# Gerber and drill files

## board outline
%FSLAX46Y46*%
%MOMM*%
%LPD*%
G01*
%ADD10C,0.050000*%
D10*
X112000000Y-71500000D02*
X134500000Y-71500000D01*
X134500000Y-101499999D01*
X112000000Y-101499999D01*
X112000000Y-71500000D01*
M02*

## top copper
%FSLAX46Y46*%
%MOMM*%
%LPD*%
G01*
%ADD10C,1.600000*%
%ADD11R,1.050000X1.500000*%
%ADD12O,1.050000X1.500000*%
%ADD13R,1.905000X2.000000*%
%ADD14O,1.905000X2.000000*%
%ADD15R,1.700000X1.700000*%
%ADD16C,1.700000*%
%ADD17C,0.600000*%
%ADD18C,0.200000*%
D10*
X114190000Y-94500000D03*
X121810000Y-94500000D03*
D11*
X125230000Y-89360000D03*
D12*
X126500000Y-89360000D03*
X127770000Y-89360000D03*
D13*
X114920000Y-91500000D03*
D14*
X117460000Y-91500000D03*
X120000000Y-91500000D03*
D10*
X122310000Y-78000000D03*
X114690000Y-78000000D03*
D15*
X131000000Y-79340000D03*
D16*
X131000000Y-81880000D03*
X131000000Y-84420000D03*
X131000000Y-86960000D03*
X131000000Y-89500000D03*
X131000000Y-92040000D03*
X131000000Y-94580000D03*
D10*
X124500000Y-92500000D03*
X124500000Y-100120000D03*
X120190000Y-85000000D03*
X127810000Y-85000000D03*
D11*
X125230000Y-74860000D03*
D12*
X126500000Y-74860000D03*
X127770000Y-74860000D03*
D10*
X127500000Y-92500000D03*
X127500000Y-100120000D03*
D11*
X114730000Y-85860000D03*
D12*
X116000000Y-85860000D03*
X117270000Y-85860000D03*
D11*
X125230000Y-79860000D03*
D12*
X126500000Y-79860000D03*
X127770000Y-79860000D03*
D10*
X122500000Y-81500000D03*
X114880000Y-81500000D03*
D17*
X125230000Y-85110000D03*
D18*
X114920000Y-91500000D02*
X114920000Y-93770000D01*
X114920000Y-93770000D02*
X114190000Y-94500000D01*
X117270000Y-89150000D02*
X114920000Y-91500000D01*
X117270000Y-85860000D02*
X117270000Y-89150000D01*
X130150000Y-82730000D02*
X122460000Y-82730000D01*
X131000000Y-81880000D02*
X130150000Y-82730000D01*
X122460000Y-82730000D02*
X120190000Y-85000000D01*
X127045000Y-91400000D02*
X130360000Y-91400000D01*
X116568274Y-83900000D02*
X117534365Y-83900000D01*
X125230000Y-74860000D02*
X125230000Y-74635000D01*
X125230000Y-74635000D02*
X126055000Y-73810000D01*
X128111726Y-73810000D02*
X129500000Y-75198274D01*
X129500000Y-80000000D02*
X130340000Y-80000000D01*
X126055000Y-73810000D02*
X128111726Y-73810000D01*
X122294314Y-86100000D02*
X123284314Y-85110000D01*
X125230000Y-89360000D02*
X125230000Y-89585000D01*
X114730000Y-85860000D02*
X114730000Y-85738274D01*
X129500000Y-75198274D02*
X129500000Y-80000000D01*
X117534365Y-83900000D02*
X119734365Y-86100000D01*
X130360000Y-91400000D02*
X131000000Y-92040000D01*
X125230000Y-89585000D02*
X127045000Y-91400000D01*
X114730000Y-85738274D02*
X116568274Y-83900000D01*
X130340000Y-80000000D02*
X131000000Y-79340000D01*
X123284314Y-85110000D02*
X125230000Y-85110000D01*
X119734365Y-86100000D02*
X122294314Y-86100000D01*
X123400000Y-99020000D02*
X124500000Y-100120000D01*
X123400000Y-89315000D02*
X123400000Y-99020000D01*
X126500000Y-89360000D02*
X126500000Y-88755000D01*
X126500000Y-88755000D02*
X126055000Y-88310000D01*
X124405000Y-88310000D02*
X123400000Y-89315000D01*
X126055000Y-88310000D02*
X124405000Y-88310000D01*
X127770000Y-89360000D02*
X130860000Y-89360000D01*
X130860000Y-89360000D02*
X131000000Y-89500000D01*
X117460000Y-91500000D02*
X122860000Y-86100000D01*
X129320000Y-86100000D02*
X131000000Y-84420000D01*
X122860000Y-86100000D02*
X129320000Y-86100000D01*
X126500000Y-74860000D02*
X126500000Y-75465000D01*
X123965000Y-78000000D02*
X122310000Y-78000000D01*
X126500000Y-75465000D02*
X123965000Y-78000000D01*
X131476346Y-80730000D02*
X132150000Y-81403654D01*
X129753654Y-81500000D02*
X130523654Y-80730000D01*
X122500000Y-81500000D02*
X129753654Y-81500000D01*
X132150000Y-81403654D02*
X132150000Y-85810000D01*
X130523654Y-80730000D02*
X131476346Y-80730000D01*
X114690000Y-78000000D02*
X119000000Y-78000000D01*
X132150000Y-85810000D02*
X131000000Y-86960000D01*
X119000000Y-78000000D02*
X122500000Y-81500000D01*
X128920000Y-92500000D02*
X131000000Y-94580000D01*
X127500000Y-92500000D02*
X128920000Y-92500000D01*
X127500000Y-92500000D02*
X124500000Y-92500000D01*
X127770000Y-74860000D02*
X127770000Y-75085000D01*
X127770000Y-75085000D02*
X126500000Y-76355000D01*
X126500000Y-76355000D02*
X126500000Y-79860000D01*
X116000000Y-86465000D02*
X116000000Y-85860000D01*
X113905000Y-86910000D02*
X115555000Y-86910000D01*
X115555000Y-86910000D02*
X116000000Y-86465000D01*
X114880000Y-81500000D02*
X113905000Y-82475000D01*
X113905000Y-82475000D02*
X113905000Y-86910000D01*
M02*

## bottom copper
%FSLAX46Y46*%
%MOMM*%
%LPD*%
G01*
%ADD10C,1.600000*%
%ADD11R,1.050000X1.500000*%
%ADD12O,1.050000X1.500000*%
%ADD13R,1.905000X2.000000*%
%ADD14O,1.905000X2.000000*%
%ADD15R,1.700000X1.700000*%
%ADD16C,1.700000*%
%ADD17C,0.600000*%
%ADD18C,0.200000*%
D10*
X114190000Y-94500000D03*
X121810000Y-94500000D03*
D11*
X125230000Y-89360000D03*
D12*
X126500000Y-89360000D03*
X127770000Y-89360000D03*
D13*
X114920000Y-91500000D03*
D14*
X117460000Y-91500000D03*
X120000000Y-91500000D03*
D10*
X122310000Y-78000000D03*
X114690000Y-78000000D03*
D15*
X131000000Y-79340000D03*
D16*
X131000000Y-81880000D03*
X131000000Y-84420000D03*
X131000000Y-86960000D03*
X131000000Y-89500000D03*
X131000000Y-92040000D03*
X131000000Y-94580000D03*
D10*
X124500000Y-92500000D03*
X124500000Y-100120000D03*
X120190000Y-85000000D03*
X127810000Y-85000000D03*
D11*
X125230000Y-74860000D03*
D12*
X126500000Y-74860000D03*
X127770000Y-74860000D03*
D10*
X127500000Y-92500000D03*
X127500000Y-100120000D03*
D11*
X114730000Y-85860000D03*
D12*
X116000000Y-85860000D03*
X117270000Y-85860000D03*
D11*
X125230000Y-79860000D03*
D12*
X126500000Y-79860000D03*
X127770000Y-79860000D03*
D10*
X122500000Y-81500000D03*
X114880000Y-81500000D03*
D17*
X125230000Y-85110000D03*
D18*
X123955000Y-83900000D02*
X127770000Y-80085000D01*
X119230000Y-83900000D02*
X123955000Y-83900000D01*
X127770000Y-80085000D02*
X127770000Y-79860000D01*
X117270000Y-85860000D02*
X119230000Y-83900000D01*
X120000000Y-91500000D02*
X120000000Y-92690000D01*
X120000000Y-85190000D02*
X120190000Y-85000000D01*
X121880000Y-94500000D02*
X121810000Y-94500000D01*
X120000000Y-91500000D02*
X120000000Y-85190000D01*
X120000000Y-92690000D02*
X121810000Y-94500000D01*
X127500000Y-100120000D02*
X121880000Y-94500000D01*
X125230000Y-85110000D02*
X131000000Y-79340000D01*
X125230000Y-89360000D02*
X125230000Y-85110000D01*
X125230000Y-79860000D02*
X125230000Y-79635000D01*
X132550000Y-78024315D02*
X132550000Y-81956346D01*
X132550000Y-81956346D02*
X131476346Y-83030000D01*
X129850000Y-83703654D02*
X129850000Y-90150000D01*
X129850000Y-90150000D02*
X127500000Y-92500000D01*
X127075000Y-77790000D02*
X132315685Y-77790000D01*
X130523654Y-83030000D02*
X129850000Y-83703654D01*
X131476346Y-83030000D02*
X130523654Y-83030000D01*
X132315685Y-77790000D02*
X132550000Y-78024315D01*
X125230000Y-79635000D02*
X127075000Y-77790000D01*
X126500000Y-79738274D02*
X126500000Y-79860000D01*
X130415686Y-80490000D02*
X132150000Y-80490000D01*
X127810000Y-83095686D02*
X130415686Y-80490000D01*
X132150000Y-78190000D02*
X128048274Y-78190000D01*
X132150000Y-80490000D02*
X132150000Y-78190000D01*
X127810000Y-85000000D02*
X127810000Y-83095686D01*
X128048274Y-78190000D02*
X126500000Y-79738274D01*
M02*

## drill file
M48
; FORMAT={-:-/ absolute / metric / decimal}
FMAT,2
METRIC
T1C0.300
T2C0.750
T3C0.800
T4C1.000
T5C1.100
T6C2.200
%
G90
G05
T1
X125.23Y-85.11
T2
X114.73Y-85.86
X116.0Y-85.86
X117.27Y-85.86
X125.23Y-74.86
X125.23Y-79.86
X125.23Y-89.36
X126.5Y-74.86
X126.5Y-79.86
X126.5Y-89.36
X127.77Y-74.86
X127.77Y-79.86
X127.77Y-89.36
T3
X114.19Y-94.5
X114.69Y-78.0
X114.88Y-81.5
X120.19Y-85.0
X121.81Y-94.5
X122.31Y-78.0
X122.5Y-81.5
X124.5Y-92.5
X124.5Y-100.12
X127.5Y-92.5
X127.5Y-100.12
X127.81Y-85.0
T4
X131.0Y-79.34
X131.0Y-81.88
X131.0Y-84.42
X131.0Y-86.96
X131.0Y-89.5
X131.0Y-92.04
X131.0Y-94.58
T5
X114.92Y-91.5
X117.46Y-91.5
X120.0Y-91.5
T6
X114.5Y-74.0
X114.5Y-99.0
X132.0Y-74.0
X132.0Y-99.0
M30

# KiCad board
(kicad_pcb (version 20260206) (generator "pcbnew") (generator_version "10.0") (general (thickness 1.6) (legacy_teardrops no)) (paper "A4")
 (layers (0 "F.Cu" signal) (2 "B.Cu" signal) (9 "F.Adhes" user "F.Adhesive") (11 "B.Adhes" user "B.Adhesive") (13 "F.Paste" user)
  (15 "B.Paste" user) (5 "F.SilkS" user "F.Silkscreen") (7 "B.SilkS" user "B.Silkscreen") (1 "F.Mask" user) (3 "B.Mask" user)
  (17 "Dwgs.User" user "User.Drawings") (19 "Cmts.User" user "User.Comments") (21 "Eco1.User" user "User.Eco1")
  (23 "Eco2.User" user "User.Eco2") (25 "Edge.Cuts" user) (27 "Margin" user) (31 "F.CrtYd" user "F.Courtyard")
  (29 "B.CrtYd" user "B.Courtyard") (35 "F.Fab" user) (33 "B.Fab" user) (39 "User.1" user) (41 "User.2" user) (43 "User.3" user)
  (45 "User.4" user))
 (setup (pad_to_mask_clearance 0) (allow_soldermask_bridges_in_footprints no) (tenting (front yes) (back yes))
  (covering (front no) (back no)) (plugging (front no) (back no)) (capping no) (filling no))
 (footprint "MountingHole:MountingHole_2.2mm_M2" (layer "F.Cu") (at 132 74)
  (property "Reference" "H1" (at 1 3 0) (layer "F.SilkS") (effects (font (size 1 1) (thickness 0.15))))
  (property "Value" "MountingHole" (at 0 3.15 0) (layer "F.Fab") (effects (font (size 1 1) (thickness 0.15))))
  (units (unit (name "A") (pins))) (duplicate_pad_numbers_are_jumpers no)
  (pad "" np_thru_hole circle (at 0 0) (size 2.2 2.2) (drill 2.2) (layers "*.Cu" "*.Mask")))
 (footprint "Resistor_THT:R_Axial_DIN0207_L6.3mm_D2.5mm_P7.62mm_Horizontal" (layer "F.Cu") (at 114.19 94.5)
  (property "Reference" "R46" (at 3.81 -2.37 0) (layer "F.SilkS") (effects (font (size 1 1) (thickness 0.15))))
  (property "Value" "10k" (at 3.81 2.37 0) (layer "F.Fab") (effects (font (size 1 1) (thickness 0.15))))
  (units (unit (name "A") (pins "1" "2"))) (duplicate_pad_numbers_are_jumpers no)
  (pad "1" thru_hole circle (at 0 0) (size 1.6 1.6) (drill 0.8) (layers "*.Cu" "*.Mask") (remove_unused_layers no) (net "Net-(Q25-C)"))
  (pad "2" thru_hole circle (at 7.62 0) (size 1.6 1.6) (drill 0.8) (layers "*.Cu" "*.Mask") (remove_unused_layers no) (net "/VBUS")))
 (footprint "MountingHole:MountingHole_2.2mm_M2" (layer "F.Cu") (at 132 99)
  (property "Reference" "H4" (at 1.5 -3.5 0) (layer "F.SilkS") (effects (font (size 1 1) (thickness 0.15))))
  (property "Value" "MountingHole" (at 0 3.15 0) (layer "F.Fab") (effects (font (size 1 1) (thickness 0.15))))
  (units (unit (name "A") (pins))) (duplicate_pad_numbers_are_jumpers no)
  (pad "" np_thru_hole circle (at 0 0) (size 2.2 2.2) (drill 2.2) (layers "*.Cu" "*.Mask")))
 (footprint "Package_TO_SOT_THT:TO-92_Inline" (layer "F.Cu") (at 125.23 89.36)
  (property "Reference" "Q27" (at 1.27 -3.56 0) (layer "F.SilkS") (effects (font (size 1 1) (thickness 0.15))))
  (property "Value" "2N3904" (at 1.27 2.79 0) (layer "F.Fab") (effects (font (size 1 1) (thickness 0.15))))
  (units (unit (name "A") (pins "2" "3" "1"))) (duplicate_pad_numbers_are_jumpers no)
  (pad "1" thru_hole rect (at 0 0) (size 1.05 1.5) (drill 0.75) (layers "*.Cu" "*.Mask") (remove_unused_layers no) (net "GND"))
  (pad "2" thru_hole oval (at 1.27 0) (size 1.05 1.5) (drill 0.75) (layers "*.Cu" "*.Mask") (remove_unused_layers no) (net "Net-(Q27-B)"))
  (pad "3" thru_hole oval (at 2.54 0) (size 1.05 1.5) (drill 0.75) (layers "*.Cu" "*.Mask") (remove_unused_layers no) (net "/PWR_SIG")))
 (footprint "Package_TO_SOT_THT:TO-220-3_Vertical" (layer "F.Cu") (at 114.92 91.5)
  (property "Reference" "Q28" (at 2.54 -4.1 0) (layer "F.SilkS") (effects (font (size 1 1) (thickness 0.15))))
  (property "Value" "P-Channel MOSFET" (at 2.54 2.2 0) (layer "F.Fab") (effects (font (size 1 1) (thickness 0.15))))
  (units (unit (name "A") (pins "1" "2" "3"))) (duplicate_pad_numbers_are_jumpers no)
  (pad "1" thru_hole rect (at 0 0) (size 1.905 2) (drill 1.1) (layers "*.Cu" "*.Mask") (remove_unused_layers no) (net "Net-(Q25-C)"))
  (pad "2" thru_hole oval (at 2.54 0) (size 1.905 2) (drill 1.1) (layers "*.Cu" "*.Mask") (remove_unused_layers no) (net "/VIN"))
  (pad "3" thru_hole oval (at 5.08 0) (size 1.905 2) (drill 1.1) (layers "*.Cu" "*.Mask") (remove_unused_layers no) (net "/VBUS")))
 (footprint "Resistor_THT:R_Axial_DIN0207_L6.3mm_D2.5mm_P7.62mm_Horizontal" (layer "F.Cu") (at 122.31 78 180)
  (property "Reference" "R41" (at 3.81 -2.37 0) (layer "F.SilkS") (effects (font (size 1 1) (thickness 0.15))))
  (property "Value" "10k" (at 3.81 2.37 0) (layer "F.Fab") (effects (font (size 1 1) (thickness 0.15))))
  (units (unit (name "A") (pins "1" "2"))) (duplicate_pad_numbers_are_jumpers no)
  (pad "1" thru_hole circle (at 0 0 180) (size 1.6 1.6) (drill 0.8) (layers "*.Cu" "*.Mask") (remove_unused_layers no) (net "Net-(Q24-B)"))
  (pad "2" thru_hole circle (at 7.62 0 180) (size 1.6 1.6) (drill 0.8) (layers "*.Cu" "*.Mask") (remove_unused_layers no) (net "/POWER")))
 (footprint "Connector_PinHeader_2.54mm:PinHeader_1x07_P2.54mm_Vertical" (layer "F.Cu") (at 131 79.34)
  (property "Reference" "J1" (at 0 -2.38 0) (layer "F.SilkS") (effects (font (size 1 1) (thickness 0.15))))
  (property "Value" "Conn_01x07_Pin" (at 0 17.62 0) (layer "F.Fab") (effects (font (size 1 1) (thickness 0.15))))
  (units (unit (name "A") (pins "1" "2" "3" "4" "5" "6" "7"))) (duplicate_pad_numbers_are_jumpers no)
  (pad "1" thru_hole rect (at 0 0) (size 1.7 1.7) (drill 1) (layers "*.Cu" "*.Mask") (remove_unused_layers no) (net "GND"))
  (pad "2" thru_hole circle (at 0 2.54) (size 1.7 1.7) (drill 1) (layers "*.Cu" "*.Mask") (remove_unused_layers no) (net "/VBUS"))
  (pad "3" thru_hole circle (at 0 5.08) (size 1.7 1.7) (drill 1) (layers "*.Cu" "*.Mask") (remove_unused_layers no) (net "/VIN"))
  (pad "4" thru_hole circle (at 0 7.62) (size 1.7 1.7) (drill 1) (layers "*.Cu" "*.Mask") (remove_unused_layers no) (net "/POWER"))
  (pad "5" thru_hole circle (at 0 10.16) (size 1.7 1.7) (drill 1) (layers "*.Cu" "*.Mask") (remove_unused_layers no) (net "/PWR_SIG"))
  (pad "6" thru_hole circle (at 0 12.7) (size 1.7 1.7) (drill 1) (layers "*.Cu" "*.Mask") (remove_unused_layers no) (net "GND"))
  (pad "7" thru_hole circle (at 0 15.24) (size 1.7 1.7) (drill 1) (layers "*.Cu" "*.Mask") (remove_unused_layers no) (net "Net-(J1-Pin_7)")))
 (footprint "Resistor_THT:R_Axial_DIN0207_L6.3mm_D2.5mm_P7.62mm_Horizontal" (layer "F.Cu") (at 124.5 92.5 -90)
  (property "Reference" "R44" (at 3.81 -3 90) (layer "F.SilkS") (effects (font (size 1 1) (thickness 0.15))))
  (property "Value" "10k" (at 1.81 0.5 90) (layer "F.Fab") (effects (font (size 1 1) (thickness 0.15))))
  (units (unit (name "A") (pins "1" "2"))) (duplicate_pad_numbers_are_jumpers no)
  (pad "1" thru_hole circle (at 0 0 270) (size 1.6 1.6) (drill 0.8) (layers "*.Cu" "*.Mask") (remove_unused_layers no)
   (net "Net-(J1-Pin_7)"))
  (pad "2" thru_hole circle (at 7.62 0 270) (size 1.6 1.6) (drill 0.8) (layers "*.Cu" "*.Mask") (remove_unused_layers no)
   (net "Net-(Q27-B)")))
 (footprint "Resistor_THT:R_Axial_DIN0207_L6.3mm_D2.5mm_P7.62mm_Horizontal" (layer "F.Cu") (at 120.19 85)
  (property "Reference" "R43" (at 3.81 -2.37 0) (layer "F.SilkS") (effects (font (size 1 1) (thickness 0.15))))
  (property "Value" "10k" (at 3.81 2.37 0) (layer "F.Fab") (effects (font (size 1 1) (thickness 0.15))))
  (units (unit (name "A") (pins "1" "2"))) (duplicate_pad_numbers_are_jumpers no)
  (pad "1" thru_hole circle (at 0 0) (size 1.6 1.6) (drill 0.8) (layers "*.Cu" "*.Mask") (remove_unused_layers no) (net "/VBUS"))
  (pad "2" thru_hole circle (at 7.62 0) (size 1.6 1.6) (drill 0.8) (layers "*.Cu" "*.Mask") (remove_unused_layers no) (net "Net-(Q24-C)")))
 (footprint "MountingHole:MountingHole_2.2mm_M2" (layer "F.Cu") (at 114.5 74)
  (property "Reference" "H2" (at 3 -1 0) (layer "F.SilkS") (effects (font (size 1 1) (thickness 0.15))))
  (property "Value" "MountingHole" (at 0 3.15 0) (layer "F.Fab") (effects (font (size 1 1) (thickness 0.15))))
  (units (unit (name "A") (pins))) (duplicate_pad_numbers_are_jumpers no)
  (pad "" np_thru_hole circle (at 0 0) (size 2.2 2.2) (drill 2.2) (layers "*.Cu" "*.Mask")))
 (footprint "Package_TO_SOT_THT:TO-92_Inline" (layer "F.Cu") (at 125.23 74.86)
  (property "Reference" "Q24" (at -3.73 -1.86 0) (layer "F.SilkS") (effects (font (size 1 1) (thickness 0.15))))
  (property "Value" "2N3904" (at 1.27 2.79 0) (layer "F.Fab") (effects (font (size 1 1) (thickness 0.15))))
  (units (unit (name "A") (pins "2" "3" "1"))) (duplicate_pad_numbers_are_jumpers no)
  (pad "1" thru_hole rect (at 0 0) (size 1.05 1.5) (drill 0.75) (layers "*.Cu" "*.Mask") (remove_unused_layers no) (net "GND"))
  (pad "2" thru_hole oval (at 1.27 0) (size 1.05 1.5) (drill 0.75) (layers "*.Cu" "*.Mask") (remove_unused_layers no) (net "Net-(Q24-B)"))
  (pad "3" thru_hole oval (at 2.54 0) (size 1.05 1.5) (drill 0.75) (layers "*.Cu" "*.Mask") (remove_unused_layers no) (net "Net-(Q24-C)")))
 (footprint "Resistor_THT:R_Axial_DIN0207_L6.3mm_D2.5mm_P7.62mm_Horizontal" (layer "F.Cu") (at 127.5 92.5 -90)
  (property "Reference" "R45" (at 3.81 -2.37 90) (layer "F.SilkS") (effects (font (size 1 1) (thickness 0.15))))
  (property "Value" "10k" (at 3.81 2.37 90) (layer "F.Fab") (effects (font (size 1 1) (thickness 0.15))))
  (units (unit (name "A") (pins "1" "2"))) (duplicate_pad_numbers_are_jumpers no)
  (pad "1" thru_hole circle (at 0 0 270) (size 1.6 1.6) (drill 0.8) (layers "*.Cu" "*.Mask") (remove_unused_layers no)
   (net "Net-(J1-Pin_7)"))
  (pad "2" thru_hole circle (at 7.62 0 270) (size 1.6 1.6) (drill 0.8) (layers "*.Cu" "*.Mask") (remove_unused_layers no) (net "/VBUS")))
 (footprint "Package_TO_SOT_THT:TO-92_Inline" (layer "F.Cu") (at 114.73 85.86)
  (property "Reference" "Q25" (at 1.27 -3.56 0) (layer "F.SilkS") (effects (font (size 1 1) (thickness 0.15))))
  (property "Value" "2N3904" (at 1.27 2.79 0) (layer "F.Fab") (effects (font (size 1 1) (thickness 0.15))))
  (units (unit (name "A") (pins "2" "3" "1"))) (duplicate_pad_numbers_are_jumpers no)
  (pad "1" thru_hole rect (at 0 0) (size 1.05 1.5) (drill 0.75) (layers "*.Cu" "*.Mask") (remove_unused_layers no) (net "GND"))
  (pad "2" thru_hole oval (at 1.27 0) (size 1.05 1.5) (drill 0.75) (layers "*.Cu" "*.Mask") (remove_unused_layers no) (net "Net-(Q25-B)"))
  (pad "3" thru_hole oval (at 2.54 0) (size 1.05 1.5) (drill 0.75) (layers "*.Cu" "*.Mask") (remove_unused_layers no) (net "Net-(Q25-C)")))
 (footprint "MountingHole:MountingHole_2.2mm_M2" (layer "F.Cu") (at 114.5 99)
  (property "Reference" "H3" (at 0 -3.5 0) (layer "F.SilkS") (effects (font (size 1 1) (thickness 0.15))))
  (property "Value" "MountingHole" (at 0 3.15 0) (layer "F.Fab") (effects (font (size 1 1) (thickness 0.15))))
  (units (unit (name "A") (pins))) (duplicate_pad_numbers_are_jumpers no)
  (pad "" np_thru_hole circle (at 0 0) (size 2.2 2.2) (drill 2.2) (layers "*.Cu" "*.Mask")))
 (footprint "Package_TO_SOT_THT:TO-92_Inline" (layer "F.Cu") (at 125.23 79.86)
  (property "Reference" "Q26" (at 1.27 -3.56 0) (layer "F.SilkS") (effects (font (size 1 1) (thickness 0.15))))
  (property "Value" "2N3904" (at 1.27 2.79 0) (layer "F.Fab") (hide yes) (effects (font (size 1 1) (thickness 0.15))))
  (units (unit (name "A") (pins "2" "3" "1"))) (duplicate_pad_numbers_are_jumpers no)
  (pad "1" thru_hole rect (at 0 0) (size 1.05 1.5) (drill 0.75) (layers "*.Cu" "*.Mask") (remove_unused_layers no) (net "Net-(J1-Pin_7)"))
  (pad "2" thru_hole oval (at 1.27 0) (size 1.05 1.5) (drill 0.75) (layers "*.Cu" "*.Mask") (remove_unused_layers no) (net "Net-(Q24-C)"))
  (pad "3" thru_hole oval (at 2.54 0) (size 1.05 1.5) (drill 0.75) (layers "*.Cu" "*.Mask") (remove_unused_layers no) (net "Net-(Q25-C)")))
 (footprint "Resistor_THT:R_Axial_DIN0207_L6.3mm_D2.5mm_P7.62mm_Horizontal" (layer "F.Cu") (at 122.5 81.5 180)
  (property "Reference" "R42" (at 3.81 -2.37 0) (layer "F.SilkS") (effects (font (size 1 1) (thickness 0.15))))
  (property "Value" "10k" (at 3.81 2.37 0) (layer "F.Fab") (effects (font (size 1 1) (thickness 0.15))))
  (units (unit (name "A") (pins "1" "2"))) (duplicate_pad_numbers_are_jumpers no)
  (pad "1" thru_hole circle (at 0 0 180) (size 1.6 1.6) (drill 0.8) (layers "*.Cu" "*.Mask") (remove_unused_layers no) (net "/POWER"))
  (pad "2" thru_hole circle (at 7.62 0 180) (size 1.6 1.6) (drill 0.8) (layers "*.Cu" "*.Mask") (remove_unused_layers no)
   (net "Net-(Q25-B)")))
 (gr_rect (start 112 71.5) (end 134.5 101.499999) (stroke (width 0.05) (type default)) (fill no) (layer "Edge.Cuts"))
 (segment (start 114.92 91.5) (end 114.92 93.77) (width 0.2) (layer "F.Cu") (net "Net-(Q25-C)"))
 (segment (start 114.92 93.77) (end 114.19 94.5) (width 0.2) (layer "F.Cu") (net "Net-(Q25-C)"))
 (segment (start 117.27 89.15) (end 114.92 91.5) (width 0.2) (layer "F.Cu") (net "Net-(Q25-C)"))
 (segment (start 117.27 85.86) (end 117.27 89.15) (width 0.2) (layer "F.Cu") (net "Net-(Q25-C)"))
 (segment (start 123.955 83.9) (end 127.77 80.085) (width 0.2) (layer "B.Cu") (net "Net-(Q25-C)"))
 (segment (start 119.23 83.9) (end 123.955 83.9) (width 0.2) (layer "B.Cu") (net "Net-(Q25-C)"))
 (segment (start 127.77 80.085) (end 127.77 79.86) (width 0.2) (layer "B.Cu") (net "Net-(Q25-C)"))
 (segment (start 117.27 85.86) (end 119.23 83.9) (width 0.2) (layer "B.Cu") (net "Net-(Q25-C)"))
 (segment (start 130.15 82.73) (end 122.46 82.73) (width 0.2) (layer "F.Cu") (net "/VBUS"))
 (segment (start 131 81.88) (end 130.15 82.73) (width 0.2) (layer "F.Cu") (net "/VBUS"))
 (segment (start 122.46 82.73) (end 120.19 85) (width 0.2) (layer "F.Cu") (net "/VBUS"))
 (segment (start 120 91.5) (end 120 92.69) (width 0.2) (layer "B.Cu") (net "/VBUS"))
 (segment (start 120 85.19) (end 120.19 85) (width 0.2) (layer "B.Cu") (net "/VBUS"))
 (segment (start 121.88 94.5) (end 121.81 94.5) (width 0.2) (layer "B.Cu") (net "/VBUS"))
 (segment (start 120 91.5) (end 120 85.19) (width 0.2) (layer "B.Cu") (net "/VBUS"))
 (segment (start 120 92.69) (end 121.81 94.5) (width 0.2) (layer "B.Cu") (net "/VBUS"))
 (segment (start 127.5 100.12) (end 121.88 94.5) (width 0.2) (layer "B.Cu") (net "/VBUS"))
 (segment (start 127.045 91.4) (end 130.36 91.4) (width 0.2) (layer "F.Cu") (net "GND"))
 (segment (start 116.568274 83.9) (end 117.534365 83.9) (width 0.2) (layer "F.Cu") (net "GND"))
 (segment (start 125.23 74.86) (end 125.23 74.635) (width 0.2) (layer "F.Cu") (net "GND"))
 (segment (start 125.23 74.635) (end 126.055 73.81) (width 0.2) (layer "F.Cu") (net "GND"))
 (segment (start 128.111726 73.81) (end 129.5 75.198274) (width 0.2) (layer "F.Cu") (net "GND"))
 (segment (start 129.5 80) (end 130.34 80) (width 0.2) (layer "F.Cu") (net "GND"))
 (segment (start 126.055 73.81) (end 128.111726 73.81) (width 0.2) (layer "F.Cu") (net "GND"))
 (segment (start 122.294314 86.1) (end 123.284314 85.11) (width 0.2) (layer "F.Cu") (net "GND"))
 (segment (start 125.23 89.36) (end 125.23 89.585) (width 0.2) (layer "F.Cu") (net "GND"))
 (segment (start 114.73 85.86) (end 114.73 85.738274) (width 0.2) (layer "F.Cu") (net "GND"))
 (segment (start 129.5 75.198274) (end 129.5 80) (width 0.2) (layer "F.Cu") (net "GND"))
 (segment (start 117.534365 83.9) (end 119.734365 86.1) (width 0.2) (layer "F.Cu") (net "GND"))
 (segment (start 130.36 91.4) (end 131 92.04) (width 0.2) (layer "F.Cu") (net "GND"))
 (segment (start 125.23 89.585) (end 127.045 91.4) (width 0.2) (layer "F.Cu") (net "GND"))
 (segment (start 114.73 85.738274) (end 116.568274 83.9) (width 0.2) (layer "F.Cu") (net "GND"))
 (segment (start 130.34 80) (end 131 79.34) (width 0.2) (layer "F.Cu") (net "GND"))
 (segment (start 123.284314 85.11) (end 125.23 85.11) (width 0.2) (layer "F.Cu") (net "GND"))
 (segment (start 119.734365 86.1) (end 122.294314 86.1) (width 0.2) (layer "F.Cu") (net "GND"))
 (via (at 125.23 85.11) (size 0.6) (drill 0.3) (layers "F.Cu" "B.Cu") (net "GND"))
 (segment (start 125.23 85.11) (end 131 79.34) (width 0.2) (layer "B.Cu") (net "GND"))
 (segment (start 125.23 89.36) (end 125.23 85.11) (width 0.2) (layer "B.Cu") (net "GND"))
 (segment (start 123.4 99.02) (end 124.5 100.12) (width 0.2) (layer "F.Cu") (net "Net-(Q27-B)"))
 (segment (start 123.4 89.315) (end 123.4 99.02) (width 0.2) (layer "F.Cu") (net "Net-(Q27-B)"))
 (segment (start 126.5 89.36) (end 126.5 88.755) (width 0.2) (layer "F.Cu") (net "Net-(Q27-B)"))
 (segment (start 126.5 88.755) (end 126.055 88.31) (width 0.2) (layer "F.Cu") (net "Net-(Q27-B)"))
 (segment (start 124.405 88.31) (end 123.4 89.315) (width 0.2) (layer "F.Cu") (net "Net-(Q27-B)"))
 (segment (start 126.055 88.31) (end 124.405 88.31) (width 0.2) (layer "F.Cu") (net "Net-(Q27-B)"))
 (segment (start 127.77 89.36) (end 130.86 89.36) (width 0.2) (layer "F.Cu") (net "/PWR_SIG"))
 (segment (start 130.86 89.36) (end 131 89.5) (width 0.2) (layer "F.Cu") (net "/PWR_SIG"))
 (segment (start 117.46 91.5) (end 122.86 86.1) (width 0.2) (layer "F.Cu") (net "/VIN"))
 (segment (start 129.32 86.1) (end 131 84.42) (width 0.2) (layer "F.Cu") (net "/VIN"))
 (segment (start 122.86 86.1) (end 129.32 86.1) (width 0.2) (layer "F.Cu") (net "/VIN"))
 (segment (start 126.5 74.86) (end 126.5 75.465) (width 0.2) (layer "F.Cu") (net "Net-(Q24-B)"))
 (segment (start 123.965 78) (end 122.31 78) (width 0.2) (layer "F.Cu") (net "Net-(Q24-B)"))
 (segment (start 126.5 75.465) (end 123.965 78) (width 0.2) (layer "F.Cu") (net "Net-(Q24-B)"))
 (segment (start 131.476346 80.73) (end 132.15 81.403654) (width 0.2) (layer "F.Cu") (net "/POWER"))
 (segment (start 129.753654 81.5) (end 130.523654 80.73) (width 0.2) (layer "F.Cu") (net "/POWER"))
 (segment (start 122.5 81.5) (end 129.753654 81.5) (width 0.2) (layer "F.Cu") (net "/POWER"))
 (segment (start 132.15 81.403654) (end 132.15 85.81) (width 0.2) (layer "F.Cu") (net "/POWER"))
 (segment (start 130.523654 80.73) (end 131.476346 80.73) (width 0.2) (layer "F.Cu") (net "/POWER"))
 (segment (start 114.69 78) (end 119 78) (width 0.2) (layer "F.Cu") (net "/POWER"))
 (segment (start 132.15 85.81) (end 131 86.96) (width 0.2) (layer "F.Cu") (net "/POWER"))
 (segment (start 119 78) (end 122.5 81.5) (width 0.2) (layer "F.Cu") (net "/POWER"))
 (segment (start 128.92 92.5) (end 131 94.58) (width 0.2) (layer "F.Cu") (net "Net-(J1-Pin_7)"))
 (segment (start 127.5 92.5) (end 128.92 92.5) (width 0.2) (layer "F.Cu") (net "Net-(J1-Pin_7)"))
 (segment (start 127.5 92.5) (end 124.5 92.5) (width 0.2) (layer "F.Cu") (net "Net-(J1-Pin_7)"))
 (segment (start 125.23 79.86) (end 125.23 79.635) (width 0.2) (layer "B.Cu") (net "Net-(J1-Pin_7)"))
 (segment (start 132.55 78.024315) (end 132.55 81.956346) (width 0.2) (layer "B.Cu") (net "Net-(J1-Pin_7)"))
 (segment (start 132.55 81.956346) (end 131.476346 83.03) (width 0.2) (layer "B.Cu") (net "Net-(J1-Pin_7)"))
 (segment (start 129.85 83.703654) (end 129.85 90.15) (width 0.2) (layer "B.Cu") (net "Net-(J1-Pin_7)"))
 (segment (start 129.85 90.15) (end 127.5 92.5) (width 0.2) (layer "B.Cu") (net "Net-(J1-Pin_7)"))
 (segment (start 127.075 77.79) (end 132.315685 77.79) (width 0.2) (layer "B.Cu") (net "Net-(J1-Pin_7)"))
 (segment (start 130.523654 83.03) (end 129.85 83.703654) (width 0.2) (layer "B.Cu") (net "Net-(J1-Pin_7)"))
 (segment (start 131.476346 83.03) (end 130.523654 83.03) (width 0.2) (layer "B.Cu") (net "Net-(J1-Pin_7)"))
 (segment (start 132.315685 77.79) (end 132.55 78.024315) (width 0.2) (layer "B.Cu") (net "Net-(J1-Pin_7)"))
 (segment (start 125.23 79.635) (end 127.075 77.79) (width 0.2) (layer "B.Cu") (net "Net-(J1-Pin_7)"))
 (segment (start 127.77 74.86) (end 127.77 75.085) (width 0.2) (layer "F.Cu") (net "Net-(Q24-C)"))
 (segment (start 127.77 75.085) (end 126.5 76.355) (width 0.2) (layer "F.Cu") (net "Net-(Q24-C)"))
 (segment (start 126.5 76.355) (end 126.5 79.86) (width 0.2) (layer "F.Cu") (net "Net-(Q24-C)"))
 (segment (start 126.5 79.738274) (end 126.5 79.86) (width 0.2) (layer "B.Cu") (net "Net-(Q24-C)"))
 (segment (start 130.415686 80.49) (end 132.15 80.49) (width 0.2) (layer "B.Cu") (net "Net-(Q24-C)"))
 (segment (start 127.81 83.095686) (end 130.415686 80.49) (width 0.2) (layer "B.Cu") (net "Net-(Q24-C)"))
 (segment (start 132.15 78.19) (end 128.048274 78.19) (width 0.2) (layer "B.Cu") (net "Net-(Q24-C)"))
 (segment (start 132.15 80.49) (end 132.15 78.19) (width 0.2) (layer "B.Cu") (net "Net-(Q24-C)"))
 (segment (start 127.81 85) (end 127.81 83.095686) (width 0.2) (layer "B.Cu") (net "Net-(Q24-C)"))
 (segment (start 128.048274 78.19) (end 126.5 79.738274) (width 0.2) (layer "B.Cu") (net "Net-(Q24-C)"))
 (segment (start 116 86.465) (end 116 85.86) (width 0.2) (layer "F.Cu") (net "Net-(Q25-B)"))
 (segment (start 113.905 86.91) (end 115.555 86.91) (width 0.2) (layer "F.Cu") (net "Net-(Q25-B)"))
 (segment (start 115.555 86.91) (end 116 86.465) (width 0.2) (layer "F.Cu") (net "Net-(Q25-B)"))
 (segment (start 114.88 81.5) (end 113.905 82.475) (width 0.2) (layer "F.Cu") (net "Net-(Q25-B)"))
 (segment (start 113.905 82.475) (end 113.905 86.91) (width 0.2) (layer "F.Cu") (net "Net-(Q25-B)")))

